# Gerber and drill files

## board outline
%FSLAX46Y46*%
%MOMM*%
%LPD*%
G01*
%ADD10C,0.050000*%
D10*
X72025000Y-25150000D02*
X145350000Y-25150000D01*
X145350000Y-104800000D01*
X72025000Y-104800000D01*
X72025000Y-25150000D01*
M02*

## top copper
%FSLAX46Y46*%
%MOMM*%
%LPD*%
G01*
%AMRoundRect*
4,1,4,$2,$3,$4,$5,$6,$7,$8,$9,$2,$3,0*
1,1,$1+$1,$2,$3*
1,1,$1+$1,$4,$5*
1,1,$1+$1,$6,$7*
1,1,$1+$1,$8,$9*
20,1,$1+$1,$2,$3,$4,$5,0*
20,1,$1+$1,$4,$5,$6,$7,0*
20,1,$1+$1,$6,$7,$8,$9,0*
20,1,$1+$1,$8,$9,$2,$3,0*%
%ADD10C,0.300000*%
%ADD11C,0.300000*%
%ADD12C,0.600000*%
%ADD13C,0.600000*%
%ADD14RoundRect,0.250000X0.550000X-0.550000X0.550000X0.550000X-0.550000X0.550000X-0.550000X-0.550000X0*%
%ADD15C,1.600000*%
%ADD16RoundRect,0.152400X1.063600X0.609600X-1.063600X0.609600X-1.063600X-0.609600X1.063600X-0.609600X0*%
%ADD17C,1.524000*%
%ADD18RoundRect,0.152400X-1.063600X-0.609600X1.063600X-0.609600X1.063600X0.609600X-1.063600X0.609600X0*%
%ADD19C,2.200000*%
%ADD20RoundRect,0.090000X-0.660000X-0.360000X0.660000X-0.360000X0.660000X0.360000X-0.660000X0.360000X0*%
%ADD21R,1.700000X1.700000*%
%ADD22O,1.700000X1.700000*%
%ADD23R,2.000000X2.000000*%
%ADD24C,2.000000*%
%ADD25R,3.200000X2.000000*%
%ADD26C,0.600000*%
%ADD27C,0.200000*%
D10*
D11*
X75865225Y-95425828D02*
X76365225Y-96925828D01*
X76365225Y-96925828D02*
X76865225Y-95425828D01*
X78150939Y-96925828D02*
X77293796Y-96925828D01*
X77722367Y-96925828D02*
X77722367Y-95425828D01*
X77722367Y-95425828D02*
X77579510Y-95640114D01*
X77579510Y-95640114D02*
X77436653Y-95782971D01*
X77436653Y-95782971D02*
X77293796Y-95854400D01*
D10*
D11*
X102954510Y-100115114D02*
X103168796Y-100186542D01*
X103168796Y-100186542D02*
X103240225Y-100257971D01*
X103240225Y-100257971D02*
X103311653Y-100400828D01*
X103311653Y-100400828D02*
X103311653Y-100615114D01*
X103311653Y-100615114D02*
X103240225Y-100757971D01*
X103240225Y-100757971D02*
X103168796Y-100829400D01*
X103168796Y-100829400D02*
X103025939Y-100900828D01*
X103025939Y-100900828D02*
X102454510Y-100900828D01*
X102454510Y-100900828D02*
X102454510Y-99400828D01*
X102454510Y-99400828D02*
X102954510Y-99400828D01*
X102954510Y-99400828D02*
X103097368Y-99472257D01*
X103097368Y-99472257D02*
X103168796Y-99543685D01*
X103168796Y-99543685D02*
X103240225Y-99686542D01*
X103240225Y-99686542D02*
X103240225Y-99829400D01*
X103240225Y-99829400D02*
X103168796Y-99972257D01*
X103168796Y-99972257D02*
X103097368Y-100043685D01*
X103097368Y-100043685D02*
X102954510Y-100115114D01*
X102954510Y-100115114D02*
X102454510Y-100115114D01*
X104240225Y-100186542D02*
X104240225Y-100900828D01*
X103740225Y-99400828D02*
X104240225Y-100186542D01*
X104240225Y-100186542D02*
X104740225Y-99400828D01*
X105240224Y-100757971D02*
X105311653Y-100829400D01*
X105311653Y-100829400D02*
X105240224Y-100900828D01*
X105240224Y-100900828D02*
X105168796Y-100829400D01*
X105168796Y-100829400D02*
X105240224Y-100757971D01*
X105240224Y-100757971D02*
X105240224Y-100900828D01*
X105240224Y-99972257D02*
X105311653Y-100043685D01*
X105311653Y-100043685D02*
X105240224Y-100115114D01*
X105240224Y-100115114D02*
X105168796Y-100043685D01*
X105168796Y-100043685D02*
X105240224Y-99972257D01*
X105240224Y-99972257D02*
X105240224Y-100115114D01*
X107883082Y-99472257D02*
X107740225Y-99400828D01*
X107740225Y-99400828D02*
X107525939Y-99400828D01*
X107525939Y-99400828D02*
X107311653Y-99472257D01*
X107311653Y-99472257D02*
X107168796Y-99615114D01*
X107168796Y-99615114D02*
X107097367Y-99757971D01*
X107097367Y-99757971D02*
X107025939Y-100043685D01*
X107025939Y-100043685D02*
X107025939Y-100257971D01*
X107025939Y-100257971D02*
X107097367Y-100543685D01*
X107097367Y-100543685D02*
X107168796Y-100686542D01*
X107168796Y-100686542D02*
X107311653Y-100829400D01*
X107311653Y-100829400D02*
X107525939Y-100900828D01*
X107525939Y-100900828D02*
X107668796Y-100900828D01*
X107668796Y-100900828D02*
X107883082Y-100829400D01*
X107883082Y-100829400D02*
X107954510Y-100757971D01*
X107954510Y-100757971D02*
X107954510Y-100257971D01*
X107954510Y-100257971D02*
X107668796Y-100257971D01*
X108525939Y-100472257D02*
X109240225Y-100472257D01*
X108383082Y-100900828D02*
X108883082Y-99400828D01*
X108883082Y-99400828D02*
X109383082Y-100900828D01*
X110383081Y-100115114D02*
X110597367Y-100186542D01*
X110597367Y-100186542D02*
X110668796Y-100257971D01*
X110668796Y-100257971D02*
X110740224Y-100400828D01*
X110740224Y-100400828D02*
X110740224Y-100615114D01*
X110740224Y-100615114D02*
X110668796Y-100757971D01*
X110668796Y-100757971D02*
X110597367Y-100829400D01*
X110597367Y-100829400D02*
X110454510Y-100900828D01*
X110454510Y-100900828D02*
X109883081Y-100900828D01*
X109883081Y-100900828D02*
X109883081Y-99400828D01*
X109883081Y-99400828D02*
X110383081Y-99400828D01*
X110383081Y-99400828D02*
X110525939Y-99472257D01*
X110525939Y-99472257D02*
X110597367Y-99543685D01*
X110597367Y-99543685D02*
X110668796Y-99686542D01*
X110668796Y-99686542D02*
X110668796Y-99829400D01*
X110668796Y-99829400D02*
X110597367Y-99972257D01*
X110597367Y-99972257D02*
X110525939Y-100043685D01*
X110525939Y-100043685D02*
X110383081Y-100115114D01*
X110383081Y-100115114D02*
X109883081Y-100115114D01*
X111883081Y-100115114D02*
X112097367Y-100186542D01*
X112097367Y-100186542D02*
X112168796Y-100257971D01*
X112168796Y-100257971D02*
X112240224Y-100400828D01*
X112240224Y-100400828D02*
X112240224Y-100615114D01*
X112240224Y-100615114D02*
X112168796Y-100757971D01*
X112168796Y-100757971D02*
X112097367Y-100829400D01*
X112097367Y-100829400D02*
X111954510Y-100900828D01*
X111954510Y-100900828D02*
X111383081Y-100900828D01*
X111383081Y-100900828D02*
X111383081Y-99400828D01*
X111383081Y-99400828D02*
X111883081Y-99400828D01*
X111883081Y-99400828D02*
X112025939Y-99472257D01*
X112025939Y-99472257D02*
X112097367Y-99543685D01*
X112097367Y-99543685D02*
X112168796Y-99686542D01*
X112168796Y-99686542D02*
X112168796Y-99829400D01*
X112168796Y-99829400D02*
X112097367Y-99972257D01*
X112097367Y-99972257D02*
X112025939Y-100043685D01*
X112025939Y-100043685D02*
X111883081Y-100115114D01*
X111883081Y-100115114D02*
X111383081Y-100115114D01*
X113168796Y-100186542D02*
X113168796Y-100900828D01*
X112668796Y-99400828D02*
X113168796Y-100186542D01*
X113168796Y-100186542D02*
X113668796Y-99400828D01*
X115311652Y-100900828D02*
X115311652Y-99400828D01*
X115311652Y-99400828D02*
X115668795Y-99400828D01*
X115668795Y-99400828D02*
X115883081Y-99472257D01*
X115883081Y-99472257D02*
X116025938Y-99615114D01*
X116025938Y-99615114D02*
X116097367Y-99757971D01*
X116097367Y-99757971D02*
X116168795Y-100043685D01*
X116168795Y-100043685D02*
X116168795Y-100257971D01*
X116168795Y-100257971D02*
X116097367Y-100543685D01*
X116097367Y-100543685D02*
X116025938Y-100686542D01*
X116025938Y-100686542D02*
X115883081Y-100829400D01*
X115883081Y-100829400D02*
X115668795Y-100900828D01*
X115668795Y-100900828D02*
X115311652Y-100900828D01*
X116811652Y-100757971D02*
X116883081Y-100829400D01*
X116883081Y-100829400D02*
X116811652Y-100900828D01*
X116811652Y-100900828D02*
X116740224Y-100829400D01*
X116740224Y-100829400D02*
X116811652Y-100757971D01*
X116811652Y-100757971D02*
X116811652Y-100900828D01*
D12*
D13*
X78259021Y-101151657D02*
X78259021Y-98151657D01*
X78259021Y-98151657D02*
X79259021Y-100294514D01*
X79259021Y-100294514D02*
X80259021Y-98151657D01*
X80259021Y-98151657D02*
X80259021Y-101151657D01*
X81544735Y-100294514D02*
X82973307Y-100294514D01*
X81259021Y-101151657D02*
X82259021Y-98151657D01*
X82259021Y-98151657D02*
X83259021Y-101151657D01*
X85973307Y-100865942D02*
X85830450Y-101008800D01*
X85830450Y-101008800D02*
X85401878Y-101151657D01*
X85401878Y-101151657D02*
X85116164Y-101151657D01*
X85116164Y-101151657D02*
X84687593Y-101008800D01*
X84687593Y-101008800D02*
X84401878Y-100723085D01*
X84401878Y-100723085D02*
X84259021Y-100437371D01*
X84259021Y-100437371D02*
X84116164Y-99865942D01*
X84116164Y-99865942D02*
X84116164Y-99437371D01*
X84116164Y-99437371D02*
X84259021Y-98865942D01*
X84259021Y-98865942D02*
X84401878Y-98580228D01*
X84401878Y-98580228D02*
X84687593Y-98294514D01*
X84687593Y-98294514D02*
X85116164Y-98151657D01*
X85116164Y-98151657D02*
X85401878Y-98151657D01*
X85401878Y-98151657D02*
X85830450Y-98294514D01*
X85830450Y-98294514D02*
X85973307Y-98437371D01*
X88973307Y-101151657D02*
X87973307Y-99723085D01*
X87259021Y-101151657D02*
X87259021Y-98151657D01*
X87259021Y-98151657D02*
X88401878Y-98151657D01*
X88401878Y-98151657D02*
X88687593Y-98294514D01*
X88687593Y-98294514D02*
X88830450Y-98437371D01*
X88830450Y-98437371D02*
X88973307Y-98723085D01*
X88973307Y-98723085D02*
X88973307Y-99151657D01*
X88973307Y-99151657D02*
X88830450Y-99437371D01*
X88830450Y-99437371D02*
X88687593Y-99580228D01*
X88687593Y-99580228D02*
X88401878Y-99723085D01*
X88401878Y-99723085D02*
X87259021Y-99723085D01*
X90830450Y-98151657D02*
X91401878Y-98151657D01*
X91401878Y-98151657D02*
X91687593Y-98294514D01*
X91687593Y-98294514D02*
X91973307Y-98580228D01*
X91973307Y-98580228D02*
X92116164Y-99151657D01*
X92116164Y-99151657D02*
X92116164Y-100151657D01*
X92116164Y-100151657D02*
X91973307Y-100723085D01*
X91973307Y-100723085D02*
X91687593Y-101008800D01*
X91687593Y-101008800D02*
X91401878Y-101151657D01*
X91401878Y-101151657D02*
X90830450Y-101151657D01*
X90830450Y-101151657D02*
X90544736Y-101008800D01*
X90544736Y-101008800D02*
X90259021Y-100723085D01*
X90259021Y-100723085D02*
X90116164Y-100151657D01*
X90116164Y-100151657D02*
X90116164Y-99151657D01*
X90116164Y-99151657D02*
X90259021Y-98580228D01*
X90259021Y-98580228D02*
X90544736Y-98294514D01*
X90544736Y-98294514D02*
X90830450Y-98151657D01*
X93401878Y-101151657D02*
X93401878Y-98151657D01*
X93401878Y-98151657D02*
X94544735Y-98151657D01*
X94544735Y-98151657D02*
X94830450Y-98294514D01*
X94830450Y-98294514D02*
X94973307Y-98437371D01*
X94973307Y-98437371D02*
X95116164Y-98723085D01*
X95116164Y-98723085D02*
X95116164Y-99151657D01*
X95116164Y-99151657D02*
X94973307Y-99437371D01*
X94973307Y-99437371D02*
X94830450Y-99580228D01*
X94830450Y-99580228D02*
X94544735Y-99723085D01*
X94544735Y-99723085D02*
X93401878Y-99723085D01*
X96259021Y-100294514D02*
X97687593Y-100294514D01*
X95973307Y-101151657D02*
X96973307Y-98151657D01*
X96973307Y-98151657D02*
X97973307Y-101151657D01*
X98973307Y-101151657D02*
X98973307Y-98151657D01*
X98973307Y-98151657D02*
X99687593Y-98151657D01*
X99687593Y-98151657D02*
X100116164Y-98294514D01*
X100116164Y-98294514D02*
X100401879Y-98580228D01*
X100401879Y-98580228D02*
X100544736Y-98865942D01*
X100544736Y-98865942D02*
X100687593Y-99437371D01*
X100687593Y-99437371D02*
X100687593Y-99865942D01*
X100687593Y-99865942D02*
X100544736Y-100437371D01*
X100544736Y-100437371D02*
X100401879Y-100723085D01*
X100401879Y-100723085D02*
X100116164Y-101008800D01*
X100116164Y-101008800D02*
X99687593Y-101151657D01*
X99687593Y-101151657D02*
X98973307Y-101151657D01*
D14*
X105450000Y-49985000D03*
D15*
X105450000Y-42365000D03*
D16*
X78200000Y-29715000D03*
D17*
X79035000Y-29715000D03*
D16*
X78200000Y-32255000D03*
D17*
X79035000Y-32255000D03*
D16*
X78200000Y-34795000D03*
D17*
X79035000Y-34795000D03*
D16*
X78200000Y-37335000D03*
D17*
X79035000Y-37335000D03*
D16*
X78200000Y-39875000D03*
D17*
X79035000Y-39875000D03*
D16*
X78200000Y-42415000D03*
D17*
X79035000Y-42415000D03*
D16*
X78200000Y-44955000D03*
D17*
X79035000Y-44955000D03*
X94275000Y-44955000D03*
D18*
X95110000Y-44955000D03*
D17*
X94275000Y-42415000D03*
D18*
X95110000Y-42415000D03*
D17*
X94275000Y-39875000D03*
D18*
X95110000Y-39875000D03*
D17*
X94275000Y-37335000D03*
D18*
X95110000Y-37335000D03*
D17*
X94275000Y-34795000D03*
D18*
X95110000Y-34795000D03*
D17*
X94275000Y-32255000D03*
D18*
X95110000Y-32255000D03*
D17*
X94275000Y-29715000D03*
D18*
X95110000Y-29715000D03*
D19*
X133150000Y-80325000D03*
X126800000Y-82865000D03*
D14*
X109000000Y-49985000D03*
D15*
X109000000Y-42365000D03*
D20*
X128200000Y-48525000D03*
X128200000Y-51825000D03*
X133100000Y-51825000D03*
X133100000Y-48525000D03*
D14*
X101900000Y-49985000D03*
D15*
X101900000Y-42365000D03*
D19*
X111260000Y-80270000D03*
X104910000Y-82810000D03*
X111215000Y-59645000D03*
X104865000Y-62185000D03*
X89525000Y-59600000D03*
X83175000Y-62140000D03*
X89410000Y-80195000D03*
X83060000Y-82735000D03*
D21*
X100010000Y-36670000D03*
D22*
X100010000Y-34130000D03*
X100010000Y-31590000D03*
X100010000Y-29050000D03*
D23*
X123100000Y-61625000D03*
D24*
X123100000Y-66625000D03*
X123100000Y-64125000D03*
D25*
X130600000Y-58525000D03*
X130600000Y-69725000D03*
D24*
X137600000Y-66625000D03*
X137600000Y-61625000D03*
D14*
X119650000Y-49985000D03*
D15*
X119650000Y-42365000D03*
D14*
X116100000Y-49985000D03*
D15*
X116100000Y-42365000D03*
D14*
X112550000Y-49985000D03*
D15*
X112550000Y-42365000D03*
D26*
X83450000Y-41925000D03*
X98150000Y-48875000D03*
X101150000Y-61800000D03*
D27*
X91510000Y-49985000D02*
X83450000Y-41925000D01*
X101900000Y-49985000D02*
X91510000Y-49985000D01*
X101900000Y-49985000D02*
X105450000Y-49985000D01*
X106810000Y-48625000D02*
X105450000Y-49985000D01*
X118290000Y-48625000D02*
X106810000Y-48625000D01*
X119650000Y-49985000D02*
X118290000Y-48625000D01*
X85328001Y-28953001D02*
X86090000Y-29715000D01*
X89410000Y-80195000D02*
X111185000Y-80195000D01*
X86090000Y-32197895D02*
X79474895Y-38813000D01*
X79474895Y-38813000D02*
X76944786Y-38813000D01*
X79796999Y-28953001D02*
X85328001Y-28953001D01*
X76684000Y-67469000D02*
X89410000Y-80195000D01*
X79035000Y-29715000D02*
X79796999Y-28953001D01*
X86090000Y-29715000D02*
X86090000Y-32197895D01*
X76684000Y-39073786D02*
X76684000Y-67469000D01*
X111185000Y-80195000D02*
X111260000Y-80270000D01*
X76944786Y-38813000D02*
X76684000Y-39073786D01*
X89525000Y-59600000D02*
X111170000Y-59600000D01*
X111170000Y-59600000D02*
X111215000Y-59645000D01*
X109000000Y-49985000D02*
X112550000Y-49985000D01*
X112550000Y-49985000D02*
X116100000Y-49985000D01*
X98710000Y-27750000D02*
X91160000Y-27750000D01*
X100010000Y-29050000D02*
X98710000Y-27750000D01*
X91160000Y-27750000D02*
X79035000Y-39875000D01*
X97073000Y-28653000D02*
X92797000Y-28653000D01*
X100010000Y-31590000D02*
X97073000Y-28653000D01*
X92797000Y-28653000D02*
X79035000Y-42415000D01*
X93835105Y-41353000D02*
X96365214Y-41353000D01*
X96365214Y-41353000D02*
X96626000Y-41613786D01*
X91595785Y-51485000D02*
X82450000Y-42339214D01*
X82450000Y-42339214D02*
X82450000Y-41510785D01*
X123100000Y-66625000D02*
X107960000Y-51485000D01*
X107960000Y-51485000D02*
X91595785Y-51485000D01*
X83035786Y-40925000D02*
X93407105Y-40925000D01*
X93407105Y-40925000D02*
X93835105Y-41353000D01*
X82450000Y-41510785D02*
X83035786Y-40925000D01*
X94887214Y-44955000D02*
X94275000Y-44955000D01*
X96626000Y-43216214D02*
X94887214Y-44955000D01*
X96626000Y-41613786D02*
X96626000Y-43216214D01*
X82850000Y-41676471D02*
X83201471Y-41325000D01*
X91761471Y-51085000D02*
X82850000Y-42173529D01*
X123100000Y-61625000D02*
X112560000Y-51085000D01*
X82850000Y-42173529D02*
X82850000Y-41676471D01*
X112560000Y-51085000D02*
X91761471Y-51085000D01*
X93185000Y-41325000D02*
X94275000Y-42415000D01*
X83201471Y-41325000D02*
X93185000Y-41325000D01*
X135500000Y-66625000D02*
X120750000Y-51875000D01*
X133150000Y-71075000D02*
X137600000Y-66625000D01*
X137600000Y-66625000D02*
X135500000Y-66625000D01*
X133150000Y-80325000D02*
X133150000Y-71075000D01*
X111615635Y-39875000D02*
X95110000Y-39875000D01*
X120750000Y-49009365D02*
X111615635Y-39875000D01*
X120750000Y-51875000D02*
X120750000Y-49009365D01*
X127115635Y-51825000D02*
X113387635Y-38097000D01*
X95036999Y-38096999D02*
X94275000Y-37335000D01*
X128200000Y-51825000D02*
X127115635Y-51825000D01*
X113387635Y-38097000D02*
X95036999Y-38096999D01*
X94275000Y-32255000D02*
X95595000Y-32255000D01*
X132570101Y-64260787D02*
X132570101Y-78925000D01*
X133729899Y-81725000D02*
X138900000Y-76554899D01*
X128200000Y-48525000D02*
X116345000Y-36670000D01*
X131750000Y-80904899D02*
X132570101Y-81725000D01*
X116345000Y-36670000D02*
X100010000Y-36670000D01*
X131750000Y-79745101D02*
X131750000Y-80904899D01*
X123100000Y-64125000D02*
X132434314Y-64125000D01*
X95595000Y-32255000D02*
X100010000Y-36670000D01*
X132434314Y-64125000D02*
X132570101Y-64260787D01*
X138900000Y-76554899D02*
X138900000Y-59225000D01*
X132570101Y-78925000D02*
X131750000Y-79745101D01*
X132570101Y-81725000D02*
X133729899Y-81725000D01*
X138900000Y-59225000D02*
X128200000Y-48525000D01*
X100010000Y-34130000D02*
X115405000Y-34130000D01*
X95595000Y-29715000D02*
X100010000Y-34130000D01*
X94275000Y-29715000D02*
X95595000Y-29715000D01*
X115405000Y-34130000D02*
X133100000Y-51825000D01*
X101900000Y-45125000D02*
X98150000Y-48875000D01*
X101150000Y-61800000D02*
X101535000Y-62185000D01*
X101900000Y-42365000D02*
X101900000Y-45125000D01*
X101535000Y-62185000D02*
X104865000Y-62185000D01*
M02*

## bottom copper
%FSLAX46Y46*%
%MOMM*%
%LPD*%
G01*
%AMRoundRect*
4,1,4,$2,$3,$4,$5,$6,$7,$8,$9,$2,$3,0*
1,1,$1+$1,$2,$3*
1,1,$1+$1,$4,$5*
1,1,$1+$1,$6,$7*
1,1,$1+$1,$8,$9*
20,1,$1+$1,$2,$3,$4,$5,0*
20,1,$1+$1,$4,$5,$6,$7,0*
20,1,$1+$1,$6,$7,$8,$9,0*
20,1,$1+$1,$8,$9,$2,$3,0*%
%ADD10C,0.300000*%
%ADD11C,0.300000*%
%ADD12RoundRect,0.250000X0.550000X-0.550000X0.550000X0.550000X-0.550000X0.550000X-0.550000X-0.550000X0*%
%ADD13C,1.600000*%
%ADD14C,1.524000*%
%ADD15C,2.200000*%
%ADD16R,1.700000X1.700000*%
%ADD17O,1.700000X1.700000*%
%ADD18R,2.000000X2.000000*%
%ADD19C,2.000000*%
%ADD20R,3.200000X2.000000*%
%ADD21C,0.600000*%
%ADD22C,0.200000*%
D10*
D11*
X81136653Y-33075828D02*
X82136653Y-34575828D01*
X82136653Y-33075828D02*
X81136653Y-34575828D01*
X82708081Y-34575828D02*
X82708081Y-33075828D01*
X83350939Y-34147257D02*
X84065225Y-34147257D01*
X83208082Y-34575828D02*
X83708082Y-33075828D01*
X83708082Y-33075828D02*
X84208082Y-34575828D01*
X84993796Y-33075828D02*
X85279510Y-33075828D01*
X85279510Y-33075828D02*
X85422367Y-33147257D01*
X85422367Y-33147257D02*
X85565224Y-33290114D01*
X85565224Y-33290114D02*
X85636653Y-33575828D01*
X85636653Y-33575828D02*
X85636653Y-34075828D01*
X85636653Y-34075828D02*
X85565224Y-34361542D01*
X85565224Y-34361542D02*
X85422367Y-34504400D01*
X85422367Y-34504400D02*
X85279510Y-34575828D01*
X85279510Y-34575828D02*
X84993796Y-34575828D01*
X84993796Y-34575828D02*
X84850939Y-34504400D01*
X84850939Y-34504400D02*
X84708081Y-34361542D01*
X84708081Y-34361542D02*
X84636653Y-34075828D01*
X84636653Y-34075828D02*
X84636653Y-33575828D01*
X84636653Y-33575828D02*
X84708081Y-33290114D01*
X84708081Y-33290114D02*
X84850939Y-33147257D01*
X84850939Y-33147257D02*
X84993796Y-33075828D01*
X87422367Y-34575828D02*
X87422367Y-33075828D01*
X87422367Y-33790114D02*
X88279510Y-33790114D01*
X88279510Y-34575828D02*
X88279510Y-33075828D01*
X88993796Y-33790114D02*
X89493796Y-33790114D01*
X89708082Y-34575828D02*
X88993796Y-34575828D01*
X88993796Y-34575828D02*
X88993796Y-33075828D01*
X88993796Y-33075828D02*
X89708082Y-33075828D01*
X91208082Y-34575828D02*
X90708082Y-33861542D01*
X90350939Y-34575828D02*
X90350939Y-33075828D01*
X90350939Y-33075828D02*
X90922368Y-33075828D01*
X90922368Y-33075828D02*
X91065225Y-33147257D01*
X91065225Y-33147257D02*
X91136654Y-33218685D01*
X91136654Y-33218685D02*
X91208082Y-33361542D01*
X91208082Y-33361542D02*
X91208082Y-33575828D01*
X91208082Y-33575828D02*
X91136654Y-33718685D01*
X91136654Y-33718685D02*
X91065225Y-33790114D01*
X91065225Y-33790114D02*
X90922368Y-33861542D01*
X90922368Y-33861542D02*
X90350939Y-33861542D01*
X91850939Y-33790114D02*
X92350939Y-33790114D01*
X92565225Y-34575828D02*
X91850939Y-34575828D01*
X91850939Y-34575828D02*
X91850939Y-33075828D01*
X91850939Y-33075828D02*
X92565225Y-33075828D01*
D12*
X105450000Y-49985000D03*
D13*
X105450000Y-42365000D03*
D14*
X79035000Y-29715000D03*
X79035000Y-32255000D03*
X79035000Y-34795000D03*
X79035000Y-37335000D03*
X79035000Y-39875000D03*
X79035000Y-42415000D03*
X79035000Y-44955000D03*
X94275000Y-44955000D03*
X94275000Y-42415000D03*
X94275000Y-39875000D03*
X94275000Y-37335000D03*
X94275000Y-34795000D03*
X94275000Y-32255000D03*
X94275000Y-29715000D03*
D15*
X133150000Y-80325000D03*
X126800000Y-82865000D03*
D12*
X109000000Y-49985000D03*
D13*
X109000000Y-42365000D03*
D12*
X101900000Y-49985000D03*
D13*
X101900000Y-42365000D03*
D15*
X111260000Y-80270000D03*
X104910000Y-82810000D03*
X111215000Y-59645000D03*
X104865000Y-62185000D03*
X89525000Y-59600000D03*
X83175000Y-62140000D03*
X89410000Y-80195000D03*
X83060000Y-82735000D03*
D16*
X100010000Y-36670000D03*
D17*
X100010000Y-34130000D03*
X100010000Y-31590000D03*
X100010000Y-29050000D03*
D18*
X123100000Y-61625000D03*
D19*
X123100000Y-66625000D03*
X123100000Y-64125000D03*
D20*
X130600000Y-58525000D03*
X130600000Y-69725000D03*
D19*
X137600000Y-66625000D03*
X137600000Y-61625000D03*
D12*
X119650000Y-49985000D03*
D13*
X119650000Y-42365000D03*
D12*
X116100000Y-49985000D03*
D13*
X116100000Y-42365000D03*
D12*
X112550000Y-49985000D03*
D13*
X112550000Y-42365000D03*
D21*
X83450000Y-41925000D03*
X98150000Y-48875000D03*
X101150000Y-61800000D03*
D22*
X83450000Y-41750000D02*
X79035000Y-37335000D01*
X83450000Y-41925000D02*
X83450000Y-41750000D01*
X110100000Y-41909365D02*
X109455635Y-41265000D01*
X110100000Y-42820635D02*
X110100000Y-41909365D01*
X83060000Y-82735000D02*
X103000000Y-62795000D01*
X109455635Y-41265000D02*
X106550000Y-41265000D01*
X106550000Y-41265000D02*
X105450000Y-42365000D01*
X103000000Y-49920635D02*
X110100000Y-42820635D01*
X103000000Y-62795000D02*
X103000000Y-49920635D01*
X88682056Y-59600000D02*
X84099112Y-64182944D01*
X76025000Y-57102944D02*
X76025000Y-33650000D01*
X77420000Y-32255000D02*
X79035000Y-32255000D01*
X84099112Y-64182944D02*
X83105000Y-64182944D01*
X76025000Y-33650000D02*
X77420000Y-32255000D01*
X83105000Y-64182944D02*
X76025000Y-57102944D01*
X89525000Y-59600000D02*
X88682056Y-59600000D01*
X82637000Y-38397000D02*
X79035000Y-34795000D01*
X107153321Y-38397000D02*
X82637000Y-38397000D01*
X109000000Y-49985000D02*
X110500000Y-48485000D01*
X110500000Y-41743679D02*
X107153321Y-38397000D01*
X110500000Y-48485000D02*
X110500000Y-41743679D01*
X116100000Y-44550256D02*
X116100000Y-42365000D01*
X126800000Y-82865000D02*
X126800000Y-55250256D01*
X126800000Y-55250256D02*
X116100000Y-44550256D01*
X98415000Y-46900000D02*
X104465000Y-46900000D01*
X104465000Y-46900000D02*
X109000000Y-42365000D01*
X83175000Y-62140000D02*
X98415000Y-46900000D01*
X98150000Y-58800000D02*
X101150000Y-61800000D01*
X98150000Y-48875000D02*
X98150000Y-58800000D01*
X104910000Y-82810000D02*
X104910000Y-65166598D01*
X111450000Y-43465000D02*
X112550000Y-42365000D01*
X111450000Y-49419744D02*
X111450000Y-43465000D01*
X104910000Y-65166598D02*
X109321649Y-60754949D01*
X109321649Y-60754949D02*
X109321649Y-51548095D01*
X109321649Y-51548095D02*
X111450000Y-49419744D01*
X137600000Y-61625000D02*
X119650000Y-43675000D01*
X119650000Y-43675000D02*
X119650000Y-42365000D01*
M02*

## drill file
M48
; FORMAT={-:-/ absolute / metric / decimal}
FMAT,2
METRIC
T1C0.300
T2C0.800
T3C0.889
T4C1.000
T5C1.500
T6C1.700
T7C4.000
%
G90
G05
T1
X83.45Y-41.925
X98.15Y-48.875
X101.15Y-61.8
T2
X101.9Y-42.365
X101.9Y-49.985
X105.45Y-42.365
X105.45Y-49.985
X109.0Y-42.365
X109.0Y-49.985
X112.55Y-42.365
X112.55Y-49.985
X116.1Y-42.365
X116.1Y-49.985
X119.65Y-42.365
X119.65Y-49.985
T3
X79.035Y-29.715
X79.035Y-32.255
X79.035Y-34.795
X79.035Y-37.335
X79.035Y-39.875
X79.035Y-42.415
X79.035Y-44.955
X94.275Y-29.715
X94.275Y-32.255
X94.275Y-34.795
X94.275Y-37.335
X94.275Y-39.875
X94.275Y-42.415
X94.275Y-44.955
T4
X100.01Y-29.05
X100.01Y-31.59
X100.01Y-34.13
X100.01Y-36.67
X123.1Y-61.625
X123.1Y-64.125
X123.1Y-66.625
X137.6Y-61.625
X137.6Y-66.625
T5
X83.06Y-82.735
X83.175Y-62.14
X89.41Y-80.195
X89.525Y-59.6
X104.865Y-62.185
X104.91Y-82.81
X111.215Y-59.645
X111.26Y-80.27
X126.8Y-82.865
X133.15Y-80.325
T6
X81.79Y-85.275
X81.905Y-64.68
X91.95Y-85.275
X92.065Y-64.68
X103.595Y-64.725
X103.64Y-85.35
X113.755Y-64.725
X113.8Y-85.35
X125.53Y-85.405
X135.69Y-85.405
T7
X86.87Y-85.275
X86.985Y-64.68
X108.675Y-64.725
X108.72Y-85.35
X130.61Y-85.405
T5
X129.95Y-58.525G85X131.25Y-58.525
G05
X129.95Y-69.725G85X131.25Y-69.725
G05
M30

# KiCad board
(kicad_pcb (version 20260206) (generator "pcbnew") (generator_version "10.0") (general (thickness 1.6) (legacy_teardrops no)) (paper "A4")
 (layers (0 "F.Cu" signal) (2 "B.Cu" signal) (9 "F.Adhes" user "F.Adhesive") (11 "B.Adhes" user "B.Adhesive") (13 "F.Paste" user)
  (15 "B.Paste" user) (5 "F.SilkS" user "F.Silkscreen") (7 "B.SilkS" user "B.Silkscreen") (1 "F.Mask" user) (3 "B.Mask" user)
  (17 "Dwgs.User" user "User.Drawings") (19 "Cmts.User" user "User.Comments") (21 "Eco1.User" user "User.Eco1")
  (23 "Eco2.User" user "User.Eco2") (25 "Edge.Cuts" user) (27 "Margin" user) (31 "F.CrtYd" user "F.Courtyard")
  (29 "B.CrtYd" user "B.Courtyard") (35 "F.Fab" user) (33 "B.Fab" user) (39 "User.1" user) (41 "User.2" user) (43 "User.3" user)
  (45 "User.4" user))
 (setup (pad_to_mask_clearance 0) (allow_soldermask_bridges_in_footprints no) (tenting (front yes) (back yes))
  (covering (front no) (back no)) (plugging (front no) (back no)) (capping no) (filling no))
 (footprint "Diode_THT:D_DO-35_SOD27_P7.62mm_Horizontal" (layer "F.Cu") (at 105.45 49.985 90)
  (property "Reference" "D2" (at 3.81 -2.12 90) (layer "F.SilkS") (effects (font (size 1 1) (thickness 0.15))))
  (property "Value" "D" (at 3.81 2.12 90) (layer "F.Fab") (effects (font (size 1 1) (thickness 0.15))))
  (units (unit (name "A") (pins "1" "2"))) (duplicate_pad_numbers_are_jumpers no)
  (pad "1" thru_hole roundrect (at 0 0 90) (size 1.6 1.6) (drill 0.8) (layers "*.Cu" "*.Mask") (remove_unused_layers no)
   (roundrect_rratio 0.15625) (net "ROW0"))
  (pad "2" thru_hole circle (at 7.62 0 90) (size 1.6 1.6) (drill 0.8) (layers "*.Cu" "*.Mask") (remove_unused_layers no) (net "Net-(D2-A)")))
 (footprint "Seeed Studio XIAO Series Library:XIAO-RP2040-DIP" (layer "F.Cu") (at 86.655 37.335 90)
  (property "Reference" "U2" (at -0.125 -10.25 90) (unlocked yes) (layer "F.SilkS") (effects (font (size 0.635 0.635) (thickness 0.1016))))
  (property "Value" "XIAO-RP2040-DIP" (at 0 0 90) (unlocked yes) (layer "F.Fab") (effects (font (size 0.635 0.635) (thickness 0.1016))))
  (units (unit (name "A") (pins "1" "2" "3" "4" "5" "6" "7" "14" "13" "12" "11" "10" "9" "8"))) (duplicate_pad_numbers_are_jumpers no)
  (pad "1" smd roundrect (at 7.62 -8.455 180) (size 2.432 1.524) (layers "F.Cu" "F.Mask") (roundrect_rratio 0.1) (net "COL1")
   (thermal_bridge_angle 45))
  (pad "1" thru_hole circle (at 7.62 -7.62 180) (size 1.524 1.524) (drill 0.889) (layers "*.Cu" "*.Mask") (remove_unused_layers no)
   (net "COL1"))
  (pad "2" smd roundrect (at 5.08 -8.455 180) (size 2.432 1.524) (layers "F.Cu" "F.Mask") (roundrect_rratio 0.1) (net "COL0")
   (thermal_bridge_angle 45))
  (pad "2" thru_hole circle (at 5.08 -7.62 180) (size 1.524 1.524) (drill 0.889) (layers "*.Cu" "*.Mask") (remove_unused_layers no)
   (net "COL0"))
  (pad "3" smd roundrect (at 2.54 -8.455 180) (size 2.432 1.524) (layers "F.Cu" "F.Mask") (roundrect_rratio 0.1) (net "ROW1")
   (thermal_bridge_angle 45))
  (pad "3" thru_hole circle (at 2.54 -7.62 180) (size 1.524 1.524) (drill 0.889) (layers "*.Cu" "*.Mask") (remove_unused_layers no)
   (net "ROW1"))
  (pad "4" smd roundrect (at 0 -8.455 180) (size 2.432 1.524) (layers "F.Cu" "F.Mask") (roundrect_rratio 0.1) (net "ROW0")
   (thermal_bridge_angle 45))
  (pad "4" thru_hole circle (at 0 -7.62 180) (size 1.524 1.524) (drill 0.889) (layers "*.Cu" "*.Mask") (remove_unused_layers no)
   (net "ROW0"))
  (pad "5" smd roundrect (at -2.54 -8.455 180) (size 2.432 1.524) (layers "F.Cu" "F.Mask") (roundrect_rratio 0.1) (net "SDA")
   (thermal_bridge_angle 45))
  (pad "5" thru_hole circle (at -2.54 -7.62 180) (size 1.524 1.524) (drill 0.889) (layers "*.Cu" "*.Mask") (remove_unused_layers no)
   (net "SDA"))
  (pad "6" smd roundrect (at -5.08 -8.455 180) (size 2.432 1.524) (layers "F.Cu" "F.Mask") (roundrect_rratio 0.1) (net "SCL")
   (thermal_bridge_angle 45))
  (pad "6" thru_hole circle (at -5.08 -7.62 180) (size 1.524 1.524) (drill 0.889) (layers "*.Cu" "*.Mask") (remove_unused_layers no)
   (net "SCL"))
  (pad "7" smd roundrect (at -7.62 -8.455 180) (size 2.432 1.524) (layers "F.Cu" "F.Mask") (roundrect_rratio 0.1)
   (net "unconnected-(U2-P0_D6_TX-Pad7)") (thermal_bridge_angle 45))
  (pad "7" thru_hole circle (at -7.62 -7.62 180) (size 1.524 1.524) (drill 0.889) (layers "*.Cu" "*.Mask") (remove_unused_layers no)
   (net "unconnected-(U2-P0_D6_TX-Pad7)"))
  (pad "8" thru_hole circle (at -7.62 7.62) (size 1.524 1.524) (drill 0.889) (layers "*.Cu" "*.Mask") (remove_unused_layers no)
   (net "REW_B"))
  (pad "8" smd roundrect (at -7.62 8.455) (size 2.432 1.524) (layers "F.Cu" "F.Mask") (roundrect_rratio 0.1) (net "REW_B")
   (thermal_bridge_angle 45))
  (pad "9" thru_hole circle (at -5.08 7.62) (size 1.524 1.524) (drill 0.889) (layers "*.Cu" "*.Mask") (remove_unused_layers no)
   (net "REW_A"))
  (pad "9" smd roundrect (at -5.08 8.455) (size 2.432 1.524) (layers "F.Cu" "F.Mask") (roundrect_rratio 0.1) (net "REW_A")
   (thermal_bridge_angle 45))
  (pad "10" thru_hole circle (at -2.54 7.62) (size 1.524 1.524) (drill 0.889) (layers "*.Cu" "*.Mask") (remove_unused_layers no)
   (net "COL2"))
  (pad "10" smd roundrect (at -2.54 8.455) (size 2.432 1.524) (layers "F.Cu" "F.Mask") (roundrect_rratio 0.1) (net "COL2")
   (thermal_bridge_angle 45))
  (pad "11" thru_hole circle (at 0 7.62) (size 1.524 1.524) (drill 0.889) (layers "*.Cu" "*.Mask") (remove_unused_layers no) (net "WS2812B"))
  (pad "11" smd roundrect (at 0 8.455) (size 2.432 1.524) (layers "F.Cu" "F.Mask") (roundrect_rratio 0.1) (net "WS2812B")
   (thermal_bridge_angle 45))
  (pad "12" thru_hole circle (at 2.54 7.62) (size 1.524 1.524) (drill 0.889) (layers "*.Cu" "*.Mask") (remove_unused_layers no)
   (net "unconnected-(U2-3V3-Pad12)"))
  (pad "12" smd roundrect (at 2.54 8.455) (size 2.432 1.524) (layers "F.Cu" "F.Mask") (roundrect_rratio 0.1)
   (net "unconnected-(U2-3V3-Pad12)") (thermal_bridge_angle 45))
  (pad "13" thru_hole circle (at 5.08 7.62) (size 1.524 1.524) (drill 0.889) (layers "*.Cu" "*.Mask") (remove_unused_layers no) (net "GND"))
  (pad "13" smd roundrect (at 5.08 8.455) (size 2.432 1.524) (layers "F.Cu" "F.Mask") (roundrect_rratio 0.1) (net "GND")
   (thermal_bridge_angle 45))
  (pad "14" thru_hole circle (at 7.62 7.62) (size 1.524 1.524) (drill 0.889) (layers "*.Cu" "*.Mask") (remove_unused_layers no) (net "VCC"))
  (pad "14" smd roundrect (at 7.62 8.455) (size 2.432 1.524) (layers "F.Cu" "F.Mask") (roundrect_rratio 0.1) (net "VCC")
   (thermal_bridge_angle 45)))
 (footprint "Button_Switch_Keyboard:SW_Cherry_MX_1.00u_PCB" (layer "F.Cu") (at 133.15 80.325)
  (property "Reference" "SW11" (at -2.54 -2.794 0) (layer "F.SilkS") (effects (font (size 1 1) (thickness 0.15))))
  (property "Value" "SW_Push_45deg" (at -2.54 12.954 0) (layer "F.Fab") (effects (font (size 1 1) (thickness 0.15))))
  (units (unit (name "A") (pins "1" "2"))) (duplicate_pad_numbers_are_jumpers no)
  (pad "" np_thru_hole circle (at -7.62 5.08) (size 1.7 1.7) (drill 1.7) (layers "*.Cu" "*.Mask"))
  (pad "" np_thru_hole circle (at -2.54 5.08) (size 4 4) (drill 4) (layers "*.Cu" "*.Mask"))
  (pad "" np_thru_hole circle (at 2.54 5.08) (size 1.7 1.7) (drill 1.7) (layers "*.Cu" "*.Mask"))
  (pad "1" thru_hole circle (at 0 0) (size 2.2 2.2) (drill 1.5) (layers "*.Cu" "*.Mask") (remove_unused_layers no) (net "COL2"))
  (pad "2" thru_hole circle (at -6.35 2.54) (size 2.2 2.2) (drill 1.5) (layers "*.Cu" "*.Mask") (remove_unused_layers no) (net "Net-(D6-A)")))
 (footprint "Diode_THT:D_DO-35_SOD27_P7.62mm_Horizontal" (layer "F.Cu") (at 109 49.985 90)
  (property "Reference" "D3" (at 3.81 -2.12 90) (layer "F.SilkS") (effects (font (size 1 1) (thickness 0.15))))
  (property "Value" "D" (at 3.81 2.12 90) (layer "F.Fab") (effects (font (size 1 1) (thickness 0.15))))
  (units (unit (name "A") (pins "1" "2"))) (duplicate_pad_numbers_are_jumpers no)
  (pad "1" thru_hole roundrect (at 0 0 90) (size 1.6 1.6) (drill 0.8) (layers "*.Cu" "*.Mask") (remove_unused_layers no)
   (roundrect_rratio 0.15625) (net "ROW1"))
  (pad "2" thru_hole circle (at 7.62 0 90) (size 1.6 1.6) (drill 0.8) (layers "*.Cu" "*.Mask") (remove_unused_layers no) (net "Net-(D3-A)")))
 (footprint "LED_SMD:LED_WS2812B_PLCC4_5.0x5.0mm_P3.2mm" (layer "F.Cu") (at 130.65 50.175)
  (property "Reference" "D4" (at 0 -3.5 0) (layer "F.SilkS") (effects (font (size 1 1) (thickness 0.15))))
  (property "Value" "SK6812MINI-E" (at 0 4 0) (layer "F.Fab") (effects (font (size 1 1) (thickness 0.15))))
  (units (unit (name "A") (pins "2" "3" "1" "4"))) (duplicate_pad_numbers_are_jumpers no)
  (pad "1" smd roundrect (at -2.45 -1.65) (size 1.5 0.9) (layers "F.Cu" "F.Mask" "F.Paste") (roundrect_rratio 0.1) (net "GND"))
  (pad "2" smd roundrect (at -2.45 1.65) (size 1.5 0.9) (layers "F.Cu" "F.Mask" "F.Paste") (roundrect_rratio 0.1) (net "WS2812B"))
  (pad "3" smd roundrect (at 2.45 1.65) (size 1.5 0.9) (layers "F.Cu" "F.Mask" "F.Paste") (roundrect_rratio 0.1) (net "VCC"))
  (pad "4" smd roundrect (at 2.45 -1.65) (size 1.5 0.9) (layers "F.Cu" "F.Mask" "F.Paste") (roundrect_rratio 0.1)
   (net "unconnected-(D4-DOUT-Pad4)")))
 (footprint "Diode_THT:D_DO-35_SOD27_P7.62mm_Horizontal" (layer "F.Cu") (at 101.9 49.985 90)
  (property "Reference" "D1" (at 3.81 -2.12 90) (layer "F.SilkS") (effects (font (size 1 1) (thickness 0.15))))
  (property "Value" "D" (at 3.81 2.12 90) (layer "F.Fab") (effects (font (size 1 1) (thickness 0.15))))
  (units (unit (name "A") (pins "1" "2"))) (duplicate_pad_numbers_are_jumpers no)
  (pad "1" thru_hole roundrect (at 0 0 90) (size 1.6 1.6) (drill 0.8) (layers "*.Cu" "*.Mask") (remove_unused_layers no)
   (roundrect_rratio 0.15625) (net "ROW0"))
  (pad "2" thru_hole circle (at 7.62 0 90) (size 1.6 1.6) (drill 0.8) (layers "*.Cu" "*.Mask") (remove_unused_layers no) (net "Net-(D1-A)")))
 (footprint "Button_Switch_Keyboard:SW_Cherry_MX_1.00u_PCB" (layer "F.Cu") (at 111.26 80.27)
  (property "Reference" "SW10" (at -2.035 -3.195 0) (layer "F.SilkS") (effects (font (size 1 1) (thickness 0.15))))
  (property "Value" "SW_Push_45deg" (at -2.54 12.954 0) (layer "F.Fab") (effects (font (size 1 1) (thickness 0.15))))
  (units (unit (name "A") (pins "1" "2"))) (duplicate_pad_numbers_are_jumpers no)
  (pad "" np_thru_hole circle (at -7.62 5.08) (size 1.7 1.7) (drill 1.7) (layers "*.Cu" "*.Mask"))
  (pad "" np_thru_hole circle (at -2.54 5.08) (size 4 4) (drill 4) (layers "*.Cu" "*.Mask"))
  (pad "" np_thru_hole circle (at 2.54 5.08) (size 1.7 1.7) (drill 1.7) (layers "*.Cu" "*.Mask"))
  (pad "1" thru_hole circle (at 0 0) (size 2.2 2.2) (drill 1.5) (layers "*.Cu" "*.Mask") (remove_unused_layers no) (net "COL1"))
  (pad "2" thru_hole circle (at -6.35 2.54) (size 2.2 2.2) (drill 1.5) (layers "*.Cu" "*.Mask") (remove_unused_layers no) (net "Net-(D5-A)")))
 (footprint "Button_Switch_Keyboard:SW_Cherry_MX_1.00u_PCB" (layer "F.Cu") (at 111.215 59.645)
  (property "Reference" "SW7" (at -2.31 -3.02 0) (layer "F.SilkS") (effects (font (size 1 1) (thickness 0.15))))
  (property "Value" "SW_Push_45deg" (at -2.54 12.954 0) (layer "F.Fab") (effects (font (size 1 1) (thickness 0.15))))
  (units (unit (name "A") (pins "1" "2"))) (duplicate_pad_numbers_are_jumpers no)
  (pad "" np_thru_hole circle (at -7.62 5.08) (size 1.7 1.7) (drill 1.7) (layers "*.Cu" "*.Mask"))
  (pad "" np_thru_hole circle (at -2.54 5.08) (size 4 4) (drill 4) (layers "*.Cu" "*.Mask"))
  (pad "" np_thru_hole circle (at 2.54 5.08) (size 1.7 1.7) (drill 1.7) (layers "*.Cu" "*.Mask"))
  (pad "1" thru_hole circle (at 0 0) (size 2.2 2.2) (drill 1.5) (layers "*.Cu" "*.Mask") (remove_unused_layers no) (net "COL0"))
  (pad "2" thru_hole circle (at -6.35 2.54) (size 2.2 2.2) (drill 1.5) (layers "*.Cu" "*.Mask") (remove_unused_layers no) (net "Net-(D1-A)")))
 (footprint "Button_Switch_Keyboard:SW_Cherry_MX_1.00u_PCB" (layer "F.Cu") (at 89.525 59.6)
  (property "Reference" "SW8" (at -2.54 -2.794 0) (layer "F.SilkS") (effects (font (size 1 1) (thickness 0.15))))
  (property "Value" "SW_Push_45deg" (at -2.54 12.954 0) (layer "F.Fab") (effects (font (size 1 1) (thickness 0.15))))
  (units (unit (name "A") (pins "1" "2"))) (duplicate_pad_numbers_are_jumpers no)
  (pad "" np_thru_hole circle (at -7.62 5.08) (size 1.7 1.7) (drill 1.7) (layers "*.Cu" "*.Mask"))
  (pad "" np_thru_hole circle (at -2.54 5.08) (size 4 4) (drill 4) (layers "*.Cu" "*.Mask"))
  (pad "" np_thru_hole circle (at 2.54 5.08) (size 1.7 1.7) (drill 1.7) (layers "*.Cu" "*.Mask"))
  (pad "1" thru_hole circle (at 0 0) (size 2.2 2.2) (drill 1.5) (layers "*.Cu" "*.Mask") (remove_unused_layers no) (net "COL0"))
  (pad "2" thru_hole circle (at -6.35 2.54) (size 2.2 2.2) (drill 1.5) (layers "*.Cu" "*.Mask") (remove_unused_layers no) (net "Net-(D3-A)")))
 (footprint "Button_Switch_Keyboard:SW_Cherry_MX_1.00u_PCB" (layer "F.Cu") (at 89.41 80.195)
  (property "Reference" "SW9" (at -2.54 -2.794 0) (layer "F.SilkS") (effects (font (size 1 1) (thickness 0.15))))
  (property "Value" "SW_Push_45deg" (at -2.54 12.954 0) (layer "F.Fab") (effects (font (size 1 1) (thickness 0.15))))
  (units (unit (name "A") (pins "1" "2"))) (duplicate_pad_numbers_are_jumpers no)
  (pad "" np_thru_hole circle (at -7.62 5.08) (size 1.7 1.7) (drill 1.7) (layers "*.Cu" "*.Mask"))
  (pad "" np_thru_hole circle (at -2.54 5.08) (size 4 4) (drill 4) (layers "*.Cu" "*.Mask"))
  (pad "" np_thru_hole circle (at 2.54 5.08) (size 1.7 1.7) (drill 1.7) (layers "*.Cu" "*.Mask"))
  (pad "1" thru_hole circle (at 0 0) (size 2.2 2.2) (drill 1.5) (layers "*.Cu" "*.Mask") (remove_unused_layers no) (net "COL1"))
  (pad "2" thru_hole circle (at -6.35 2.54) (size 2.2 2.2) (drill 1.5) (layers "*.Cu" "*.Mask") (remove_unused_layers no) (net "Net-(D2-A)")))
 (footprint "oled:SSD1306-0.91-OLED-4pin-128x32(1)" (layer "F.Cu") (at 136.51 38.86 180)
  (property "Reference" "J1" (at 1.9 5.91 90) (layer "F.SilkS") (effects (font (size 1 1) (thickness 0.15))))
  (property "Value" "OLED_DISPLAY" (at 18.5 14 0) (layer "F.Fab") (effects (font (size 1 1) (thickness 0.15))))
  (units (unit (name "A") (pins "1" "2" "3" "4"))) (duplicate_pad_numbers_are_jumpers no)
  (pad "1" thru_hole rect (at 36.5 2.19 180) (size 1.7 1.7) (drill 1) (layers "*.Cu" "*.Mask") (remove_unused_layers no) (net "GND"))
  (pad "2" thru_hole oval (at 36.5 4.73 180) (size 1.7 1.7) (drill 1) (layers "*.Cu" "*.Mask") (remove_unused_layers no) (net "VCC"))
  (pad "3" thru_hole oval (at 36.5 7.27 180) (size 1.7 1.7) (drill 1) (layers "*.Cu" "*.Mask") (remove_unused_layers no) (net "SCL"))
  (pad "4" thru_hole oval (at 36.5 9.81 180) (size 1.7 1.7) (drill 1) (layers "*.Cu" "*.Mask") (remove_unused_layers no) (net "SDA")))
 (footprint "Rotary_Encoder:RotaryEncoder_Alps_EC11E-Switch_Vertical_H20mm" (layer "F.Cu") (at 123.1 61.625)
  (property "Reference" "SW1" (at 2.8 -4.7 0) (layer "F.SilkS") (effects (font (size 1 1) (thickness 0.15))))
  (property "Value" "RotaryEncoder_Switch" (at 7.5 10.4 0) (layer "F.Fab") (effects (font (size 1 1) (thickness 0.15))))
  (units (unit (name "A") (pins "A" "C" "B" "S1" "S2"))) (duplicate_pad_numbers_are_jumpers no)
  (pad "A" thru_hole rect (at 0 0) (size 2 2) (drill 1) (layers "*.Cu" "*.Mask") (remove_unused_layers no) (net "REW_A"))
  (pad "B" thru_hole circle (at 0 5) (size 2 2) (drill 1) (layers "*.Cu" "*.Mask") (remove_unused_layers no) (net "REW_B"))
  (pad "C" thru_hole circle (at 0 2.5) (size 2 2) (drill 1) (layers "*.Cu" "*.Mask") (remove_unused_layers no) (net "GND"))
  (pad "MP" thru_hole rect (at 7.5 -3.1) (size 3.2 2) (drill oval 2.8 1.5) (layers "*.Cu" "*.Mask") (remove_unused_layers no))
  (pad "MP" thru_hole rect (at 7.5 8.1) (size 3.2 2) (drill oval 2.8 1.5) (layers "*.Cu" "*.Mask") (remove_unused_layers no))
  (pad "S1" thru_hole circle (at 14.5 5) (size 2 2) (drill 1) (layers "*.Cu" "*.Mask") (remove_unused_layers no) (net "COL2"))
  (pad "S2" thru_hole circle (at 14.5 0) (size 2 2) (drill 1) (layers "*.Cu" "*.Mask") (remove_unused_layers no) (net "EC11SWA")))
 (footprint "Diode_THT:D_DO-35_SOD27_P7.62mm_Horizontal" (layer "F.Cu") (at 119.65 49.985 90)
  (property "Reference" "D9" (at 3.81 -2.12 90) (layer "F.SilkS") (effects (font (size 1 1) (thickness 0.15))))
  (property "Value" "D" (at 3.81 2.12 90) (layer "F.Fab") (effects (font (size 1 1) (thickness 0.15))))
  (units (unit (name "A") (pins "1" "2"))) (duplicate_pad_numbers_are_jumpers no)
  (pad "1" thru_hole roundrect (at 0 0 90) (size 1.6 1.6) (drill 0.8) (layers "*.Cu" "*.Mask") (remove_unused_layers no)
   (roundrect_rratio 0.15625) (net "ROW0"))
  (pad "2" thru_hole circle (at 7.62 0 90) (size 1.6 1.6) (drill 0.8) (layers "*.Cu" "*.Mask") (remove_unused_layers no) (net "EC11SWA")))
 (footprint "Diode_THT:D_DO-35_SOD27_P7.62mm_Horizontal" (layer "F.Cu") (at 116.1 49.985 90)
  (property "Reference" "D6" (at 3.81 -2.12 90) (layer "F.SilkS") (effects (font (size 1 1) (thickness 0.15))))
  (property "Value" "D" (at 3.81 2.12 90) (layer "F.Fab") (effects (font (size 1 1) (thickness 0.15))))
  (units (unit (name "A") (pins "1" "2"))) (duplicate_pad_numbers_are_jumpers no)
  (pad "1" thru_hole roundrect (at 0 0 90) (size 1.6 1.6) (drill 0.8) (layers "*.Cu" "*.Mask") (remove_unused_layers no)
   (roundrect_rratio 0.15625) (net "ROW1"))
  (pad "2" thru_hole circle (at 7.62 0 90) (size 1.6 1.6) (drill 0.8) (layers "*.Cu" "*.Mask") (remove_unused_layers no) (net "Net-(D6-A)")))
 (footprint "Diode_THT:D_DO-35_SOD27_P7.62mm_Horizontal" (layer "F.Cu") (at 112.55 49.985 90)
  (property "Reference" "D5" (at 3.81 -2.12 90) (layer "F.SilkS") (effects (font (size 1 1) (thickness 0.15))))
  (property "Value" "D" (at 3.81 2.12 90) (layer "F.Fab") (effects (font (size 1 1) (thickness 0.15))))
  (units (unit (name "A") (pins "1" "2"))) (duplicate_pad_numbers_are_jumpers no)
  (pad "1" thru_hole roundrect (at 0 0 90) (size 1.6 1.6) (drill 0.8) (layers "*.Cu" "*.Mask") (remove_unused_layers no)
   (roundrect_rratio 0.15625) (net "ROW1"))
  (pad "2" thru_hole circle (at 7.62 0 90) (size 1.6 1.6) (drill 0.8) (layers "*.Cu" "*.Mask") (remove_unused_layers no) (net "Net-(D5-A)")))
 (gr_rect (start 72.025 25.15) (end 145.35 104.8) (stroke (width 0.05) (type default)) (fill no) (layer "Edge.Cuts"))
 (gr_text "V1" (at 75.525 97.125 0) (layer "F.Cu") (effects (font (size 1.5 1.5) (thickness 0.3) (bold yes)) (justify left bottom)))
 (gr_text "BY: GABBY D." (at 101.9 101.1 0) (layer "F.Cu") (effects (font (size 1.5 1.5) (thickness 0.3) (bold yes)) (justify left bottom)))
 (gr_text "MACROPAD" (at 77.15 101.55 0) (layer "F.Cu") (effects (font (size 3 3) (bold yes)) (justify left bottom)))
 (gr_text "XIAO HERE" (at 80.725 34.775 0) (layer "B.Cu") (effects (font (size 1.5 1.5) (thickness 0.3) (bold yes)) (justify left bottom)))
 (segment (start 91.51 49.985) (end 83.45 41.925) (width 0.2) (layer "F.Cu") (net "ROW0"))
 (segment (start 101.9 49.985) (end 91.51 49.985) (width 0.2) (layer "F.Cu") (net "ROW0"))
 (segment (start 101.9 49.985) (end 105.45 49.985) (width 0.2) (layer "F.Cu") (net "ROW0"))
 (segment (start 106.81 48.625) (end 105.45 49.985) (width 0.2) (layer "F.Cu") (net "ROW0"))
 (segment (start 118.29 48.625) (end 106.81 48.625) (width 0.2) (layer "F.Cu") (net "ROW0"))
 (segment (start 119.65 49.985) (end 118.29 48.625) (width 0.2) (layer "F.Cu") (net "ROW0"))
 (via (at 83.45 41.925) (size 0.6) (drill 0.3) (layers "F.Cu" "B.Cu") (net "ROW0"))
 (segment (start 83.45 41.75) (end 79.035 37.335) (width 0.2) (layer "B.Cu") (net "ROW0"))
 (segment (start 83.45 41.925) (end 83.45 41.75) (width 0.2) (layer "B.Cu") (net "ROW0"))
 (segment (start 110.1 41.909365) (end 109.455635 41.265) (width 0.2) (layer "B.Cu") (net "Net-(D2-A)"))
 (segment (start 110.1 42.820635) (end 110.1 41.909365) (width 0.2) (layer "B.Cu") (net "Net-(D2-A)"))
 (segment (start 83.06 82.735) (end 103 62.795) (width 0.2) (layer "B.Cu") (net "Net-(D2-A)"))
 (segment (start 109.455635 41.265) (end 106.55 41.265) (width 0.2) (layer "B.Cu") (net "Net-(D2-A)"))
 (segment (start 106.55 41.265) (end 105.45 42.365) (width 0.2) (layer "B.Cu") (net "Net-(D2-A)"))
 (segment (start 103 49.920635) (end 110.1 42.820635) (width 0.2) (layer "B.Cu") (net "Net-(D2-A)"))
 (segment (start 103 62.795) (end 103 49.920635) (width 0.2) (layer "B.Cu") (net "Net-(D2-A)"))
 (segment (start 85.328001 28.953001) (end 86.09 29.715) (width 0.2) (layer "F.Cu") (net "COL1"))
 (segment (start 89.41 80.195) (end 111.185 80.195) (width 0.2) (layer "F.Cu") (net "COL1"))
 (segment (start 86.09 32.197895) (end 79.474895 38.813) (width 0.2) (layer "F.Cu") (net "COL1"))
 (segment (start 79.474895 38.813) (end 76.944786 38.813) (width 0.2) (layer "F.Cu") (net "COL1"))
 (segment (start 79.796999 28.953001) (end 85.328001 28.953001) (width 0.2) (layer "F.Cu") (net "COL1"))
 (segment (start 76.684 67.469) (end 89.41 80.195) (width 0.2) (layer "F.Cu") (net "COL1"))
 (segment (start 79.035 29.715) (end 79.796999 28.953001) (width 0.2) (layer "F.Cu") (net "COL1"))
 (segment (start 86.09 29.715) (end 86.09 32.197895) (width 0.2) (layer "F.Cu") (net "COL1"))
 (segment (start 76.684 39.073786) (end 76.684 67.469) (width 0.2) (layer "F.Cu") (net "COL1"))
 (segment (start 111.185 80.195) (end 111.26 80.27) (width 0.2) (layer "F.Cu") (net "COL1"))
 (segment (start 76.944786 38.813) (end 76.684 39.073786) (width 0.2) (layer "F.Cu") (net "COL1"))
 (segment (start 89.525 59.6) (end 111.17 59.6) (width 0.2) (layer "F.Cu") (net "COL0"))
 (segment (start 111.17 59.6) (end 111.215 59.645) (width 0.2) (layer "F.Cu") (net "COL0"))
 (segment (start 88.682056 59.6) (end 84.099112 64.182944) (width 0.2) (layer "B.Cu") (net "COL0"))
 (segment (start 76.025 57.102944) (end 76.025 33.65) (width 0.2) (layer "B.Cu") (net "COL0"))
 (segment (start 77.42 32.255) (end 79.035 32.255) (width 0.2) (layer "B.Cu") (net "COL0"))
 (segment (start 84.099112 64.182944) (end 83.105 64.182944) (width 0.2) (layer "B.Cu") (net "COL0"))
 (segment (start 76.025 33.65) (end 77.42 32.255) (width 0.2) (layer "B.Cu") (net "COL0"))
 (segment (start 83.105 64.182944) (end 76.025 57.102944) (width 0.2) (layer "B.Cu") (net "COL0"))
 (segment (start 89.525 59.6) (end 88.682056 59.6) (width 0.2) (layer "B.Cu") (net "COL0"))
 (segment (start 109 49.985) (end 112.55 49.985) (width 0.2) (layer "F.Cu") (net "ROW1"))
 (segment (start 112.55 49.985) (end 116.1 49.985) (width 0.2) (layer "F.Cu") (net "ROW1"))
 (segment (start 82.637 38.397) (end 79.035 34.795) (width 0.2) (layer "B.Cu") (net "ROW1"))
 (segment (start 107.153321 38.397) (end 82.637 38.397) (width 0.2) (layer "B.Cu") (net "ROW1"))
 (segment (start 109 49.985) (end 110.5 48.485) (width 0.2) (layer "B.Cu") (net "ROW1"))
 (segment (start 110.5 41.743679) (end 107.153321 38.397) (width 0.2) (layer "B.Cu") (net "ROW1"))
 (segment (start 110.5 48.485) (end 110.5 41.743679) (width 0.2) (layer "B.Cu") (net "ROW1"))
 (segment (start 98.71 27.75) (end 91.16 27.75) (width 0.2) (layer "F.Cu") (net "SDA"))
 (segment (start 100.01 29.05) (end 98.71 27.75) (width 0.2) (layer "F.Cu") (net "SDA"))
 (segment (start 91.16 27.75) (end 79.035 39.875) (width 0.2) (layer "F.Cu") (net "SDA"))
 (segment (start 97.073 28.653) (end 92.797 28.653) (width 0.2) (layer "F.Cu") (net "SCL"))
 (segment (start 100.01 31.59) (end 97.073 28.653) (width 0.2) (layer "F.Cu") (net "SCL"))
 (segment (start 92.797 28.653) (end 79.035 42.415) (width 0.2) (layer "F.Cu") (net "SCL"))
 (segment (start 93.835105 41.353) (end 96.365214 41.353) (width 0.2) (layer "F.Cu") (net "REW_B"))
 (segment (start 96.365214 41.353) (end 96.626 41.613786) (width 0.2) (layer "F.Cu") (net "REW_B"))
 (segment (start 91.595785 51.485) (end 82.45 42.339214) (width 0.2) (layer "F.Cu") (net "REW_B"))
 (segment (start 82.45 42.339214) (end 82.45 41.510785) (width 0.2) (layer "F.Cu") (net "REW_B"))
 (segment (start 123.1 66.625) (end 107.96 51.485) (width 0.2) (layer "F.Cu") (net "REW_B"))
 (segment (start 107.96 51.485) (end 91.595785 51.485) (width 0.2) (layer "F.Cu") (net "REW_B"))
 (segment (start 83.035786 40.925) (end 93.407105 40.925) (width 0.2) (layer "F.Cu") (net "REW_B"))
 (segment (start 93.407105 40.925) (end 93.835105 41.353) (width 0.2) (layer "F.Cu") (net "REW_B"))
 (segment (start 82.45 41.510785) (end 83.035786 40.925) (width 0.2) (layer "F.Cu") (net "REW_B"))
 (segment (start 94.887214 44.955) (end 94.275 44.955) (width 0.2) (layer "F.Cu") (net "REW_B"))
 (segment (start 96.626 43.216214) (end 94.887214 44.955) (width 0.2) (layer "F.Cu") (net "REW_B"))
 (segment (start 96.626 41.613786) (end 96.626 43.216214) (width 0.2) (layer "F.Cu") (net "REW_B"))
 (segment (start 82.85 41.676471) (end 83.201471 41.325) (width 0.2) (layer "F.Cu") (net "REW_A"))
 (segment (start 91.761471 51.085) (end 82.85 42.173529) (width 0.2) (layer "F.Cu") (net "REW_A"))
 (segment (start 123.1 61.625) (end 112.56 51.085) (width 0.2) (layer "F.Cu") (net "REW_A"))
 (segment (start 82.85 42.173529) (end 82.85 41.676471) (width 0.2) (layer "F.Cu") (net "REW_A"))
 (segment (start 112.56 51.085) (end 91.761471 51.085) (width 0.2) (layer "F.Cu") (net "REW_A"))
 (segment (start 93.185 41.325) (end 94.275 42.415) (width 0.2) (layer "F.Cu") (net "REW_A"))
 (segment (start 83.201471 41.325) (end 93.185 41.325) (width 0.2) (layer "F.Cu") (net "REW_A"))
 (segment (start 135.5 66.625) (end 120.75 51.875) (width 0.2) (layer "F.Cu") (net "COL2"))
 (segment (start 133.15 71.075) (end 137.6 66.625) (width 0.2) (layer "F.Cu") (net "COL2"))
 (segment (start 137.6 66.625) (end 135.5 66.625) (width 0.2) (layer "F.Cu") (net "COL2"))
 (segment (start 133.15 80.325) (end 133.15 71.075) (width 0.2) (layer "F.Cu") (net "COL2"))
 (segment (start 111.615635 39.875) (end 95.11 39.875) (width 0.2) (layer "F.Cu") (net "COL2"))
 (segment (start 120.75 49.009365) (end 111.615635 39.875) (width 0.2) (layer "F.Cu") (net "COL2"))
 (segment (start 120.75 51.875) (end 120.75 49.009365) (width 0.2) (layer "F.Cu") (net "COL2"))
 (segment (start 127.115635 51.825) (end 113.387635 38.097) (width 0.2) (layer "F.Cu") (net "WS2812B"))
 (segment (start 95.036999 38.096999) (end 94.275 37.335) (width 0.2) (layer "F.Cu") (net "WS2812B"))
 (segment (start 128.2 51.825) (end 127.115635 51.825) (width 0.2) (layer "F.Cu") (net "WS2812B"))
 (segment (start 113.387635 38.097) (end 95.036999 38.096999) (width 0.2) (layer "F.Cu") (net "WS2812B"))
 (segment (start 94.275 32.255) (end 95.595 32.255) (width 0.2) (layer "F.Cu") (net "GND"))
 (segment (start 132.570101 64.260787) (end 132.570101 78.925) (width 0.2) (layer "F.Cu") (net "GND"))
 (segment (start 133.729899 81.725) (end 138.9 76.554899) (width 0.2) (layer "F.Cu") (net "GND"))
 (segment (start 128.2 48.525) (end 116.345 36.67) (width 0.2) (layer "F.Cu") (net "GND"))
 (segment (start 131.75 80.904899) (end 132.570101 81.725) (width 0.2) (layer "F.Cu") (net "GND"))
 (segment (start 116.345 36.67) (end 100.01 36.67) (width 0.2) (layer "F.Cu") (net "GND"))
 (segment (start 131.75 79.745101) (end 131.75 80.904899) (width 0.2) (layer "F.Cu") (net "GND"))
 (segment (start 123.1 64.125) (end 132.434314 64.125) (width 0.2) (layer "F.Cu") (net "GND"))
 (segment (start 95.595 32.255) (end 100.01 36.67) (width 0.2) (layer "F.Cu") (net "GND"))
 (segment (start 132.434314 64.125) (end 132.570101 64.260787) (width 0.2) (layer "F.Cu") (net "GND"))
 (segment (start 138.9 76.554899) (end 138.9 59.225) (width 0.2) (layer "F.Cu") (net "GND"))
 (segment (start 132.570101 78.925) (end 131.75 79.745101) (width 0.2) (layer "F.Cu") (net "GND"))
 (segment (start 132.570101 81.725) (end 133.729899 81.725) (width 0.2) (layer "F.Cu") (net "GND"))
 (segment (start 138.9 59.225) (end 128.2 48.525) (width 0.2) (layer "F.Cu") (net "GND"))
 (segment (start 100.01 34.13) (end 115.405 34.13) (width 0.2) (layer "F.Cu") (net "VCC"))
 (segment (start 95.595 29.715) (end 100.01 34.13) (width 0.2) (layer "F.Cu") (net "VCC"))
 (segment (start 94.275 29.715) (end 95.595 29.715) (width 0.2) (layer "F.Cu") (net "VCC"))
 (segment (start 115.405 34.13) (end 133.1 51.825) (width 0.2) (layer "F.Cu") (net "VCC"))
 (segment (start 116.1 44.550256) (end 116.1 42.365) (width 0.2) (layer "B.Cu") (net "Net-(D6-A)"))
 (segment (start 126.8 82.865) (end 126.8 55.250256) (width 0.2) (layer "B.Cu") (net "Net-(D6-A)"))
 (segment (start 126.8 55.250256) (end 116.1 44.550256) (width 0.2) (layer "B.Cu") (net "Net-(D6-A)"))
 (segment (start 98.415 46.9) (end 104.465 46.9) (width 0.2) (layer "B.Cu") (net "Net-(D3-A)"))
 (segment (start 104.465 46.9) (end 109 42.365) (width 0.2) (layer "B.Cu") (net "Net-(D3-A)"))
 (segment (start 83.175 62.14) (end 98.415 46.9) (width 0.2) (layer "B.Cu") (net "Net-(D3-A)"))
 (segment (start 101.9 45.125) (end 98.15 48.875) (width 0.2) (layer "F.Cu") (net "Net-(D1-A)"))
 (segment (start 101.15 61.8) (end 101.535 62.185) (width 0.2) (layer "F.Cu") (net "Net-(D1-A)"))
 (segment (start 101.9 42.365) (end 101.9 45.125) (width 0.2) (layer "F.Cu") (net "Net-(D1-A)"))
 (segment (start 101.535 62.185) (end 104.865 62.185) (width 0.2) (layer "F.Cu") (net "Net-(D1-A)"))
 (via (at 98.15 48.875) (size 0.6) (drill 0.3) (layers "F.Cu" "B.Cu") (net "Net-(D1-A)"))
 (via (at 101.15 61.8) (size 0.6) (drill 0.3) (layers "F.Cu" "B.Cu") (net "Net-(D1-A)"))
 (segment (start 98.15 58.8) (end 101.15 61.8) (width 0.2) (layer "B.Cu") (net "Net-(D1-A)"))
 (segment (start 98.15 48.875) (end 98.15 58.8) (width 0.2) (layer "B.Cu") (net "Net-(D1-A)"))
 (segment (start 104.91 82.81) (end 104.91 65.166598) (width 0.2) (layer "B.Cu") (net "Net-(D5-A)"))
 (segment (start 111.45 43.465) (end 112.55 42.365) (width 0.2) (layer "B.Cu") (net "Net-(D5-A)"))
 (segment (start 111.45 49.419744) (end 111.45 43.465) (width 0.2) (layer "B.Cu") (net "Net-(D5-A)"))
 (segment (start 104.91 65.166598) (end 109.321649 60.754949) (width 0.2) (layer "B.Cu") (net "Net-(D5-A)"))
 (segment (start 109.321649 60.754949) (end 109.321649 51.548095) (width 0.2) (layer "B.Cu") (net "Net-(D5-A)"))
 (segment (start 109.321649 51.548095) (end 111.45 49.419744) (width 0.2) (layer "B.Cu") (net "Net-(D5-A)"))
 (segment (start 137.6 61.625) (end 119.65 43.675) (width 0.2) (layer "B.Cu") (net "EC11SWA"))
 (segment (start 119.65 43.675) (end 119.65 42.365) (width 0.2) (layer "B.Cu") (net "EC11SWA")))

